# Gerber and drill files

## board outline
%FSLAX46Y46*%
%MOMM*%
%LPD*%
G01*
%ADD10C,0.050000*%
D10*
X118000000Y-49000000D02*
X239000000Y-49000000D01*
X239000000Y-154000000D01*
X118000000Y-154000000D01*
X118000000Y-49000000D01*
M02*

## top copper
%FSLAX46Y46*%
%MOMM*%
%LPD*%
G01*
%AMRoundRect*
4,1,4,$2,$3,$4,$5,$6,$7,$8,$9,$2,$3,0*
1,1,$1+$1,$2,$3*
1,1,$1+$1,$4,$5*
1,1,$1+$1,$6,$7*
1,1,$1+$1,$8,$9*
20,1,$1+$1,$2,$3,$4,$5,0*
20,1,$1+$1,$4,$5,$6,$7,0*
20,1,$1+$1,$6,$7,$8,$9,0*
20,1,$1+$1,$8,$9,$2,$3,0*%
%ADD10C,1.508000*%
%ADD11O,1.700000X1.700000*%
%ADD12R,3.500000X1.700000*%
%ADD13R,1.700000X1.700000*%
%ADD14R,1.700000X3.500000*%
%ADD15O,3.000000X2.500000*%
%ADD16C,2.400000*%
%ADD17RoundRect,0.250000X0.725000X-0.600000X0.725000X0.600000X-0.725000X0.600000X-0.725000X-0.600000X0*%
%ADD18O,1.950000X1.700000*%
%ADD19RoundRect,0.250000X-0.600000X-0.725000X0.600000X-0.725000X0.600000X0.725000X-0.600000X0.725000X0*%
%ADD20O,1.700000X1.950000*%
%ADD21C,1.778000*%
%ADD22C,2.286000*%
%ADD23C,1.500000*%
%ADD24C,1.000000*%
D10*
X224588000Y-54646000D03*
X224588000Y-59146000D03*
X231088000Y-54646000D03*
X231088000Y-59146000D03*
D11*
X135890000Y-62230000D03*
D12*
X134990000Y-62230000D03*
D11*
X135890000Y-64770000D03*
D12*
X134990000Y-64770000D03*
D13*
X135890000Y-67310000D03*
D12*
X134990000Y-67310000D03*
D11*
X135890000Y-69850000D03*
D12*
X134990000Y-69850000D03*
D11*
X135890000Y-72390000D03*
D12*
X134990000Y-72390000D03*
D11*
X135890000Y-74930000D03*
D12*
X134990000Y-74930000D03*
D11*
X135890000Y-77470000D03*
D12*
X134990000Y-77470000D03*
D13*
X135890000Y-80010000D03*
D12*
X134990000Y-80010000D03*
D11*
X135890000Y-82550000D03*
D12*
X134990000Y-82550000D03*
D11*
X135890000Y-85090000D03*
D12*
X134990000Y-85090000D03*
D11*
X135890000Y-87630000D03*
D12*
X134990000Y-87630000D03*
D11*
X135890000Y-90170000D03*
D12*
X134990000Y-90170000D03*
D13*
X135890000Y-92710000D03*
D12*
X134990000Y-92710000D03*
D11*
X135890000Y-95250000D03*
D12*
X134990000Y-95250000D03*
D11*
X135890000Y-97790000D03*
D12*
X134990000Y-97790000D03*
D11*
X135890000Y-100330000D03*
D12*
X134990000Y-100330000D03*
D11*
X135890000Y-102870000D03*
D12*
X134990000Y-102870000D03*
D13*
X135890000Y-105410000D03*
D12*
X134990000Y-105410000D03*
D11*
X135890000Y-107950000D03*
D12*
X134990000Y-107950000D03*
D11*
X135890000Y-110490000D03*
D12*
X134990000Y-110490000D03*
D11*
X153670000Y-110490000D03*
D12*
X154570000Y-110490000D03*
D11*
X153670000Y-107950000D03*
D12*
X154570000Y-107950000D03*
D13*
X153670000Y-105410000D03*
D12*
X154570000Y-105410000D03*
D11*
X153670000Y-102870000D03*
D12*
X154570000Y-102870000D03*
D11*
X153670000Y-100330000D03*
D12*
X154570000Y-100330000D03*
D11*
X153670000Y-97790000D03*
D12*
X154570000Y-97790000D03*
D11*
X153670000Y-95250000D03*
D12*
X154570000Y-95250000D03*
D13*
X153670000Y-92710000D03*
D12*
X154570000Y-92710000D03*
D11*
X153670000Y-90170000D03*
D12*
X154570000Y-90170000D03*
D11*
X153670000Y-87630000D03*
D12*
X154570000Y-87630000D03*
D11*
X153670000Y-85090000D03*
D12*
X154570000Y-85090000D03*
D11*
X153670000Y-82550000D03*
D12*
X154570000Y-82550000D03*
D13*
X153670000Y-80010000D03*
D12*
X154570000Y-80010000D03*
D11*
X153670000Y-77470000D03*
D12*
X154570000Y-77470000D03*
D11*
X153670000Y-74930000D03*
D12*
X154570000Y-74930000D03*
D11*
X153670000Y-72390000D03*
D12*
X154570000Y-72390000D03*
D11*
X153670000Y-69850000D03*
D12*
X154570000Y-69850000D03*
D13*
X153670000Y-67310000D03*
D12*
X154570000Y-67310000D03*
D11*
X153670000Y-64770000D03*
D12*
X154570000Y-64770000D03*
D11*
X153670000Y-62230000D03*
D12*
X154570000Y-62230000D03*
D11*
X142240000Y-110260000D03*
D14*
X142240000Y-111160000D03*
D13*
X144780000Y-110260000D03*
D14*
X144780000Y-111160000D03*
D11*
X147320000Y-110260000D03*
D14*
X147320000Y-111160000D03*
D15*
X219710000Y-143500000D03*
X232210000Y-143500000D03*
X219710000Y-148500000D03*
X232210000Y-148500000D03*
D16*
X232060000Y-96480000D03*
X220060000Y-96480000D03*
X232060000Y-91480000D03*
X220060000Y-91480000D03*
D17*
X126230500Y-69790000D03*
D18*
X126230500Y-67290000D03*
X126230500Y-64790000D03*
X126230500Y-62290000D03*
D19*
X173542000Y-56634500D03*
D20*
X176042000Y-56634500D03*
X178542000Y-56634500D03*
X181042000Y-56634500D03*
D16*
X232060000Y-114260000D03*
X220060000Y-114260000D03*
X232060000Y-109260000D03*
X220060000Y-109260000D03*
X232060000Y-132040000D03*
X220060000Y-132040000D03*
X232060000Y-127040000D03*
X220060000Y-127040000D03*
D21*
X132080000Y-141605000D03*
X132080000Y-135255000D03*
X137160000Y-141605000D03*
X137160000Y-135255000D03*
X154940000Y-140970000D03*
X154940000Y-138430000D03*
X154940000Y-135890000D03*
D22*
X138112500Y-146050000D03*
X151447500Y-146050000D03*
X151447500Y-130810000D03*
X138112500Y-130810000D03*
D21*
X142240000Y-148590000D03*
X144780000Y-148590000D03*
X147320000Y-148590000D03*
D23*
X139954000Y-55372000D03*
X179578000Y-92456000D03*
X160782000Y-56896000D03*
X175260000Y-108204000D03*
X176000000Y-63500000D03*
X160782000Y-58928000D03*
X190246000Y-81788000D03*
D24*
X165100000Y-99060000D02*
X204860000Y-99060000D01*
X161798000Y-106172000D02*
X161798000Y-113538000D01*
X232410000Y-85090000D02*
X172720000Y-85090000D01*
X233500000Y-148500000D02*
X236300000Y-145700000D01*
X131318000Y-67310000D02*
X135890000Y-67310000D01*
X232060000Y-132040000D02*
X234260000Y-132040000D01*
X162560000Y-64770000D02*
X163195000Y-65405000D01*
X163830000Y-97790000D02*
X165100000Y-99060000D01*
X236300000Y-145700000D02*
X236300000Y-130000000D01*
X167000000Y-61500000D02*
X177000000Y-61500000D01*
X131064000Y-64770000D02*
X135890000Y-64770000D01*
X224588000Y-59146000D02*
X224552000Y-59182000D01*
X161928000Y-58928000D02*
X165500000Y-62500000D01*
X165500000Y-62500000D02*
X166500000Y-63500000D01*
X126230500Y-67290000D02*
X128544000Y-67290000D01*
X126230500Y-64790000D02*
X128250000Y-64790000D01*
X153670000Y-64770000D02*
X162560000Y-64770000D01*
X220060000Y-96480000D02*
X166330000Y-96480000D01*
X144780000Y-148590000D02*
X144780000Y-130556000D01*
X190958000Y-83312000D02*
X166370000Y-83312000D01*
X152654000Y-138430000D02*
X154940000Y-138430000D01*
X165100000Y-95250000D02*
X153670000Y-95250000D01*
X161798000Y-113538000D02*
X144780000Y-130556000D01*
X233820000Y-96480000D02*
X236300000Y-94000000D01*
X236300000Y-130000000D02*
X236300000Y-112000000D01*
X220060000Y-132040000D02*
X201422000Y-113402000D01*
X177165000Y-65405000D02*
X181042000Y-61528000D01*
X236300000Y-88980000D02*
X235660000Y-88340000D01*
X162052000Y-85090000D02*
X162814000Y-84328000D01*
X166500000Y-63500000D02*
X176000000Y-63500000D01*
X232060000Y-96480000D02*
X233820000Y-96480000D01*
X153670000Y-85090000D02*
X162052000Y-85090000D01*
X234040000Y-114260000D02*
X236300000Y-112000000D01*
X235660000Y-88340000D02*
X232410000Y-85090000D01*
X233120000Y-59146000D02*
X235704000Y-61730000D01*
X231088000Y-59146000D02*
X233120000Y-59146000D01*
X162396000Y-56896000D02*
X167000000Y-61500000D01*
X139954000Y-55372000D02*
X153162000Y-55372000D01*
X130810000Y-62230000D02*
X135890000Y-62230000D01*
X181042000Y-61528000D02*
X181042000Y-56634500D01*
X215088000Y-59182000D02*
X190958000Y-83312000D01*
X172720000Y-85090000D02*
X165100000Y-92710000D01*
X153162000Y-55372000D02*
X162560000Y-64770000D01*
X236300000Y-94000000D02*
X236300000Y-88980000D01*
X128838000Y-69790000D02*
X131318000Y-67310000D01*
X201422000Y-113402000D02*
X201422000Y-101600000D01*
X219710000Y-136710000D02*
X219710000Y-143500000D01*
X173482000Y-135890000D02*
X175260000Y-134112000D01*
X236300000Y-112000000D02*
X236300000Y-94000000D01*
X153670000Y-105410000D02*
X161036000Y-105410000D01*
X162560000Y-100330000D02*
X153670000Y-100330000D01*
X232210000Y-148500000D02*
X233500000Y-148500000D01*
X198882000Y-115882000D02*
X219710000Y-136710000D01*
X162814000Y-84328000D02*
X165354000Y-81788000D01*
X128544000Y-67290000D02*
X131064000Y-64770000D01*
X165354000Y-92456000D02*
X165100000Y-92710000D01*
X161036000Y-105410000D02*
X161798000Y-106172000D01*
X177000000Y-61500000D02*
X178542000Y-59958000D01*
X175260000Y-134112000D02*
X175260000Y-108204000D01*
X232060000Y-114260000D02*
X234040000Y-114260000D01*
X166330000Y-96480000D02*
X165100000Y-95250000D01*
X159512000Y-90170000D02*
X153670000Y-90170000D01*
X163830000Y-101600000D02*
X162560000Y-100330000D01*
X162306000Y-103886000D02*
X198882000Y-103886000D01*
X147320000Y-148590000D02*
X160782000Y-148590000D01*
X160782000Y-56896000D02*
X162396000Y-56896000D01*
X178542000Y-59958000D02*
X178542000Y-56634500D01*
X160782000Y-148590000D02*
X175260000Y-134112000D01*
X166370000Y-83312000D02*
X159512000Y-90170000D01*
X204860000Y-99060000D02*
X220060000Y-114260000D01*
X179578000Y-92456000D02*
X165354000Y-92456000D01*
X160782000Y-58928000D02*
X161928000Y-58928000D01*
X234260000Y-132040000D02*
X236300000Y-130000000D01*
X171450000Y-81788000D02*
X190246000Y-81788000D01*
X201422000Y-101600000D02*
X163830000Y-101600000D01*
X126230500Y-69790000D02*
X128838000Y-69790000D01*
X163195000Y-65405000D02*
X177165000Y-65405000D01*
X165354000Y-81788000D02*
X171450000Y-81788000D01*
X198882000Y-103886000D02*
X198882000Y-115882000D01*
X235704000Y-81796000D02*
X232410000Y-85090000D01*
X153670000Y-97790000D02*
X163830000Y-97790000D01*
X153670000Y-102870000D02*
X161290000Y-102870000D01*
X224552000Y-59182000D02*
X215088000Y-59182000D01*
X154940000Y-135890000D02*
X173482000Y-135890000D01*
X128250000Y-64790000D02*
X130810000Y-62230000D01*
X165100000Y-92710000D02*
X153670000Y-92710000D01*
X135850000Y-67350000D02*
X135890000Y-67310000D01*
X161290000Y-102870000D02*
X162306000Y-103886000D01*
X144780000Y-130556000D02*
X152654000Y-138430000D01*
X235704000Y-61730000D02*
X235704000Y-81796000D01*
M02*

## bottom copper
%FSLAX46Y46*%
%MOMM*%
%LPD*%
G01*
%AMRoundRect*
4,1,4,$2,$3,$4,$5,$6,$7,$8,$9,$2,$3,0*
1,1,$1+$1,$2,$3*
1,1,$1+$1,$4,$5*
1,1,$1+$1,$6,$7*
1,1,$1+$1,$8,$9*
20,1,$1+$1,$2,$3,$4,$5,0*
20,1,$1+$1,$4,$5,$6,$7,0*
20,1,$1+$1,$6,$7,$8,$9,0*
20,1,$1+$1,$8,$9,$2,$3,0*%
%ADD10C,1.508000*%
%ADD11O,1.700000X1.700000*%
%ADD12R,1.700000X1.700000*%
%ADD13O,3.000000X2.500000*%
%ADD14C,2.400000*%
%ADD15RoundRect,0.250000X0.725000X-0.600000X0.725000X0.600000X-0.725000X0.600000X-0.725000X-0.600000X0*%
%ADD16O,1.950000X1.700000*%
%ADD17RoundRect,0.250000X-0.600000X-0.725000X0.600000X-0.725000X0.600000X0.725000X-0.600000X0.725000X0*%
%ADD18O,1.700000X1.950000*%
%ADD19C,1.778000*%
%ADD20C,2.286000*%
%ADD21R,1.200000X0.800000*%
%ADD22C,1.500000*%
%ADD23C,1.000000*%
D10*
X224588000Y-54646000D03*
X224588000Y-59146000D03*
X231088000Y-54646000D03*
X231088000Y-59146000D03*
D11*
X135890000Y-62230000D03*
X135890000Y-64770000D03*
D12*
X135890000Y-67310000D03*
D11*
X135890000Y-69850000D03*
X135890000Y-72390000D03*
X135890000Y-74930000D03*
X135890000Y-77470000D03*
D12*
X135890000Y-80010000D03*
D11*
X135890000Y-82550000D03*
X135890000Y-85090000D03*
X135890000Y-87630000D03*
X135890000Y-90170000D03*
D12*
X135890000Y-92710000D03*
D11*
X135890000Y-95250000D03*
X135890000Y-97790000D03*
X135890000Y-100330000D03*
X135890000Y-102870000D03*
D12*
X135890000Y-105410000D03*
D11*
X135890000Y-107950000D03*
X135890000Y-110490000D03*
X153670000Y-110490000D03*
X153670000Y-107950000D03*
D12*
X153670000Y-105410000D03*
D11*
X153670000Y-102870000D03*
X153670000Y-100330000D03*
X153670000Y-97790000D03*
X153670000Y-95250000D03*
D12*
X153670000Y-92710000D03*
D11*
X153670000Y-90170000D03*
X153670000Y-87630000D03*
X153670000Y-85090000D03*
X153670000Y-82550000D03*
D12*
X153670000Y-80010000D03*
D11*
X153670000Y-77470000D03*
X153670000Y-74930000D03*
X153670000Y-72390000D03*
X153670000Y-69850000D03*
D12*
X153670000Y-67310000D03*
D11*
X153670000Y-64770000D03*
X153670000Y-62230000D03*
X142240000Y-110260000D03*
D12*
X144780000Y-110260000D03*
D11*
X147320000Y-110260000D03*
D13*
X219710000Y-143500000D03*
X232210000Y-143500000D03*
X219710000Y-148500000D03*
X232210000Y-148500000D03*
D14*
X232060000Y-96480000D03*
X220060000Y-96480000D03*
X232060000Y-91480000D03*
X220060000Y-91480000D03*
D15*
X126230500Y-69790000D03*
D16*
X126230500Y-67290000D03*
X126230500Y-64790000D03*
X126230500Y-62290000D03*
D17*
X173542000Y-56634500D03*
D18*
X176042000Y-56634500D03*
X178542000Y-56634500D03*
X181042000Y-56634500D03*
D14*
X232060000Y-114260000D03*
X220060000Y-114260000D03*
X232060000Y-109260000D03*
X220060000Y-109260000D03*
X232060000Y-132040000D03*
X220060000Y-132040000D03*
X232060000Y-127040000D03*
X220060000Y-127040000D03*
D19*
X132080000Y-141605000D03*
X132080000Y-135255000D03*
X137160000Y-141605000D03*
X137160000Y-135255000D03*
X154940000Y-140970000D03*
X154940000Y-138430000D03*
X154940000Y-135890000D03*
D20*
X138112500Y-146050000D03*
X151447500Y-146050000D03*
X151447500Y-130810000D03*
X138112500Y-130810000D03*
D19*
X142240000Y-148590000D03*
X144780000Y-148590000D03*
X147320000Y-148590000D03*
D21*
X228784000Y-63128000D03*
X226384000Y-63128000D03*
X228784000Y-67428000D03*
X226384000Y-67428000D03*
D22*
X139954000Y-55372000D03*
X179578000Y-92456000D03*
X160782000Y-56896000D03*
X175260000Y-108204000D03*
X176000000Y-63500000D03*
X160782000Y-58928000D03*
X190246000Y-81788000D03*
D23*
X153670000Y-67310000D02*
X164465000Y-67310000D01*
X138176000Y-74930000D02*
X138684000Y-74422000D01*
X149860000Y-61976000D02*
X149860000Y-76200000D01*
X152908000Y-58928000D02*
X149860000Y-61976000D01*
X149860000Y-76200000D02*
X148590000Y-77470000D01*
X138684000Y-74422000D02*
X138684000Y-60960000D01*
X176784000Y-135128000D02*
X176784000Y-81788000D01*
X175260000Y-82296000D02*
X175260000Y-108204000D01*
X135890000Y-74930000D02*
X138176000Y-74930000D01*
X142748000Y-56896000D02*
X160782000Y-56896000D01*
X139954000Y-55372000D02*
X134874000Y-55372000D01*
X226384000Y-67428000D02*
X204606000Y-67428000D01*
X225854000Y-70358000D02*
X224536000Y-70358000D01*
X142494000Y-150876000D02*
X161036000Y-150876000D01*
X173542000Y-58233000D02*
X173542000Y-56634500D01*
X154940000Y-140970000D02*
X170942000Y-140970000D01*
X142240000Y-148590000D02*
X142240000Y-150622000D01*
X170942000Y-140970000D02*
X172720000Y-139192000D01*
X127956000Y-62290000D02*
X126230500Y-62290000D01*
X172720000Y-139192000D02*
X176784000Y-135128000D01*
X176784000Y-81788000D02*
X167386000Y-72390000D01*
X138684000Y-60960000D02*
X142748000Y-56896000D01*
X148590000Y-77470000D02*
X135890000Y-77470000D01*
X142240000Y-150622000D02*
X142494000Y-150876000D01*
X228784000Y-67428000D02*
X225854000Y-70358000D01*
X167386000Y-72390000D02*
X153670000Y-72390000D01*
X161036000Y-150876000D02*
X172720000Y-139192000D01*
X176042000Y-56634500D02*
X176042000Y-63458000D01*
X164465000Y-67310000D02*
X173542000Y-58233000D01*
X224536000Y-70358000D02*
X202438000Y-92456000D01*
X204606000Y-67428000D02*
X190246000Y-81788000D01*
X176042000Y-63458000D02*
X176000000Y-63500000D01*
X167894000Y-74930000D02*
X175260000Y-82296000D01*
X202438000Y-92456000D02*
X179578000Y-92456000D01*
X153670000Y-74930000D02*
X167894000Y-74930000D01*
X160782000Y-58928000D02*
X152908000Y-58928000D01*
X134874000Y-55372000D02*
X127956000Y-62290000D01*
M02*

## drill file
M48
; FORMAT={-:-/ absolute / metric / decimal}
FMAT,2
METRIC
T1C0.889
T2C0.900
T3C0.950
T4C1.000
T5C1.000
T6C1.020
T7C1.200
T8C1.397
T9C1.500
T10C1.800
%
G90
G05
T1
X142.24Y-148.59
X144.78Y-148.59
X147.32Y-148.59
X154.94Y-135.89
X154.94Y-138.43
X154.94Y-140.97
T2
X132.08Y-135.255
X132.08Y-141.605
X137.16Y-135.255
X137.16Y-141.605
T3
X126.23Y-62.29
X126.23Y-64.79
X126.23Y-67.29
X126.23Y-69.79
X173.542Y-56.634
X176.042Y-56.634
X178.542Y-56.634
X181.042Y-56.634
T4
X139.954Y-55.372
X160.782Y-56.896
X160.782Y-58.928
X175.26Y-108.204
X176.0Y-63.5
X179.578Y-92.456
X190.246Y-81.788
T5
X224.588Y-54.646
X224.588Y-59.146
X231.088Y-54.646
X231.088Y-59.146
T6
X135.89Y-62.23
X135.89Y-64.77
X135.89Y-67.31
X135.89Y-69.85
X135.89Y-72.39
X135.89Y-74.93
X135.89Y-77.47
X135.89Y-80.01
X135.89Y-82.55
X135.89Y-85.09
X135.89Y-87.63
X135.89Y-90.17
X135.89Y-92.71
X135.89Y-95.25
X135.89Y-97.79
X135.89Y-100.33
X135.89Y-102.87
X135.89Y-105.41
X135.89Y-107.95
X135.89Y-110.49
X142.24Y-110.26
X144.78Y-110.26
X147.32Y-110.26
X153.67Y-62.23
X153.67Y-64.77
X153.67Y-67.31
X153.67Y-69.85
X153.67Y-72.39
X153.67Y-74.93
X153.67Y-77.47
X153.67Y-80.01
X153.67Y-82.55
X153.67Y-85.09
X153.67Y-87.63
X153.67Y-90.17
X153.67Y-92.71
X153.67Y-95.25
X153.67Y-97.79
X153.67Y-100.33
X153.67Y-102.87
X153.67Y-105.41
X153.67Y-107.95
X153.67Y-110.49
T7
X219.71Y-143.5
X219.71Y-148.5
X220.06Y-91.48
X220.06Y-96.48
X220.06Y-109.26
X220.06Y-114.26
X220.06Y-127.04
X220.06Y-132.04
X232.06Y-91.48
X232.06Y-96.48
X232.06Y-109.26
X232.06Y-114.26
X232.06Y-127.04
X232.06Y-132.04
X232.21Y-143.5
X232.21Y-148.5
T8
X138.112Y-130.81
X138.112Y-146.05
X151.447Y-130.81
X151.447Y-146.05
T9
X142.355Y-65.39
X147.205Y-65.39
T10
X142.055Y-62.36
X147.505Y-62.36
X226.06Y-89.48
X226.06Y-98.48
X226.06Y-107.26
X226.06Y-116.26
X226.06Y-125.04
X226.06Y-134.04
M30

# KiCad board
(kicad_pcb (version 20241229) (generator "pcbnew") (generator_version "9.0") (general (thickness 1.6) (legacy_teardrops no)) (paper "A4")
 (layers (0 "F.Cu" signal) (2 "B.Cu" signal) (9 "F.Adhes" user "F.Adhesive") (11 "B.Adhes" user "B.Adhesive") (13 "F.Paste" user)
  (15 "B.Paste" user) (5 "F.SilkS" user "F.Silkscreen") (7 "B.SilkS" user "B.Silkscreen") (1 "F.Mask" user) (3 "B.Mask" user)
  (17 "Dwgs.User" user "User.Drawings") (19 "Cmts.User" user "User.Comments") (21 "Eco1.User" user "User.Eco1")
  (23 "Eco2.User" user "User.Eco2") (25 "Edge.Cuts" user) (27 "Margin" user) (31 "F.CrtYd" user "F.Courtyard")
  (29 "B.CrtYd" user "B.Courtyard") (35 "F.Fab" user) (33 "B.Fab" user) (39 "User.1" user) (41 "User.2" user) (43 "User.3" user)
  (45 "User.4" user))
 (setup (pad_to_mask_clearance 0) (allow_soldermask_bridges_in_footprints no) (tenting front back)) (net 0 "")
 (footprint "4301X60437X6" (layer "F.Cu") (at 227.838 56.896)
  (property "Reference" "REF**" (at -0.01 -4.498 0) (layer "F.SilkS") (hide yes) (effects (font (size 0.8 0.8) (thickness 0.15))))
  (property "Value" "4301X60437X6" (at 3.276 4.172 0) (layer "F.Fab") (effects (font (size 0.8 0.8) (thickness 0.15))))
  (pad "1" thru_hole circle (at -3.25 -2.25) (size 1.508 1.508) (drill 1) (layers "*.Cu" "*.Mask") (remove_unused_layers no)
   (solder_mask_margin 0.102))
  (pad "2" thru_hole circle (at -3.25 2.25) (size 1.508 1.508) (drill 1) (layers "*.Cu" "*.Mask") (remove_unused_layers no)
   (solder_mask_margin 0.102))
  (pad "3" thru_hole circle (at 3.25 -2.25) (size 1.508 1.508) (drill 1) (layers "*.Cu" "*.Mask") (remove_unused_layers no)
   (solder_mask_margin 0.102))
  (pad "4" thru_hole circle (at 3.25 2.25) (size 1.508 1.508) (drill 1) (layers "*.Cu" "*.Mask") (remove_unused_layers no)
   (solder_mask_margin 0.102)))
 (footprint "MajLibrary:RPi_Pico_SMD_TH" (layer "F.Cu") (at 144.78 86.36)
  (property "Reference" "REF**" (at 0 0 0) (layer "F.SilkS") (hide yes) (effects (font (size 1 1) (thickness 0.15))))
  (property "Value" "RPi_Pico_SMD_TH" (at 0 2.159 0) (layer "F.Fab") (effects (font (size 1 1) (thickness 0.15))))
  (pad "" np_thru_hole oval (at -2.725 -24) (size 1.8 1.8) (drill 1.8) (layers "*.Cu" "*.Mask"))
  (pad "" np_thru_hole oval (at -2.425 -20.97) (size 1.5 1.5) (drill 1.5) (layers "*.Cu" "*.Mask"))
  (pad "" np_thru_hole oval (at 2.425 -20.97) (size 1.5 1.5) (drill 1.5) (layers "*.Cu" "*.Mask"))
  (pad "" np_thru_hole oval (at 2.725 -24) (size 1.8 1.8) (drill 1.8) (layers "*.Cu" "*.Mask"))
  (pad "1" thru_hole oval (at -8.89 -24.13) (size 1.7 1.7) (drill 1.02) (layers "*.Cu" "*.Mask") (remove_unused_layers no))
  (pad "1" smd rect (at -8.89 -24.13) (size 3.5 1.7) (drill (offset -0.9 0)) (layers "F.Cu" "F.Mask"))
  (pad "2" thru_hole oval (at -8.89 -21.59) (size 1.7 1.7) (drill 1.02) (layers "*.Cu" "*.Mask") (remove_unused_layers no))
  (pad "2" smd rect (at -8.89 -21.59) (size 3.5 1.7) (drill (offset -0.9 0)) (layers "F.Cu" "F.Mask"))
  (pad "3" thru_hole rect (at -8.89 -19.05) (size 1.7 1.7) (drill 1.02) (layers "*.Cu" "*.Mask") (remove_unused_layers no))
  (pad "3" smd rect (at -8.89 -19.05) (size 3.5 1.7) (drill (offset -0.9 0)) (layers "F.Cu" "F.Mask"))
  (pad "4" thru_hole oval (at -8.89 -16.51) (size 1.7 1.7) (drill 1.02) (layers "*.Cu" "*.Mask") (remove_unused_layers no))
  (pad "4" smd rect (at -8.89 -16.51) (size 3.5 1.7) (drill (offset -0.9 0)) (layers "F.Cu" "F.Mask"))
  (pad "5" thru_hole oval (at -8.89 -13.97) (size 1.7 1.7) (drill 1.02) (layers "*.Cu" "*.Mask") (remove_unused_layers no))
  (pad "5" smd rect (at -8.89 -13.97) (size 3.5 1.7) (drill (offset -0.9 0)) (layers "F.Cu" "F.Mask"))
  (pad "6" thru_hole oval (at -8.89 -11.43) (size 1.7 1.7) (drill 1.02) (layers "*.Cu" "*.Mask") (remove_unused_layers no))
  (pad "6" smd rect (at -8.89 -11.43) (size 3.5 1.7) (drill (offset -0.9 0)) (layers "F.Cu" "F.Mask"))
  (pad "7" thru_hole oval (at -8.89 -8.89) (size 1.7 1.7) (drill 1.02) (layers "*.Cu" "*.Mask") (remove_unused_layers no))
  (pad "7" smd rect (at -8.89 -8.89) (size 3.5 1.7) (drill (offset -0.9 0)) (layers "F.Cu" "F.Mask"))
  (pad "8" thru_hole rect (at -8.89 -6.35) (size 1.7 1.7) (drill 1.02) (layers "*.Cu" "*.Mask") (remove_unused_layers no))
  (pad "8" smd rect (at -8.89 -6.35) (size 3.5 1.7) (drill (offset -0.9 0)) (layers "F.Cu" "F.Mask"))
  (pad "9" thru_hole oval (at -8.89 -3.81) (size 1.7 1.7) (drill 1.02) (layers "*.Cu" "*.Mask") (remove_unused_layers no))
  (pad "9" smd rect (at -8.89 -3.81) (size 3.5 1.7) (drill (offset -0.9 0)) (layers "F.Cu" "F.Mask"))
  (pad "10" thru_hole oval (at -8.89 -1.27) (size 1.7 1.7) (drill 1.02) (layers "*.Cu" "*.Mask") (remove_unused_layers no))
  (pad "10" smd rect (at -8.89 -1.27) (size 3.5 1.7) (drill (offset -0.9 0)) (layers "F.Cu" "F.Mask"))
  (pad "11" thru_hole oval (at -8.89 1.27) (size 1.7 1.7) (drill 1.02) (layers "*.Cu" "*.Mask") (remove_unused_layers no))
  (pad "11" smd rect (at -8.89 1.27) (size 3.5 1.7) (drill (offset -0.9 0)) (layers "F.Cu" "F.Mask"))
  (pad "12" thru_hole oval (at -8.89 3.81) (size 1.7 1.7) (drill 1.02) (layers "*.Cu" "*.Mask") (remove_unused_layers no))
  (pad "12" smd rect (at -8.89 3.81) (size 3.5 1.7) (drill (offset -0.9 0)) (layers "F.Cu" "F.Mask"))
  (pad "13" thru_hole rect (at -8.89 6.35) (size 1.7 1.7) (drill 1.02) (layers "*.Cu" "*.Mask") (remove_unused_layers no))
  (pad "13" smd rect (at -8.89 6.35) (size 3.5 1.7) (drill (offset -0.9 0)) (layers "F.Cu" "F.Mask"))
  (pad "14" thru_hole oval (at -8.89 8.89) (size 1.7 1.7) (drill 1.02) (layers "*.Cu" "*.Mask") (remove_unused_layers no))
  (pad "14" smd rect (at -8.89 8.89) (size 3.5 1.7) (drill (offset -0.9 0)) (layers "F.Cu" "F.Mask"))
  (pad "15" thru_hole oval (at -8.89 11.43) (size 1.7 1.7) (drill 1.02) (layers "*.Cu" "*.Mask") (remove_unused_layers no))
  (pad "15" smd rect (at -8.89 11.43) (size 3.5 1.7) (drill (offset -0.9 0)) (layers "F.Cu" "F.Mask"))
  (pad "16" thru_hole oval (at -8.89 13.97) (size 1.7 1.7) (drill 1.02) (layers "*.Cu" "*.Mask") (remove_unused_layers no))
  (pad "16" smd rect (at -8.89 13.97) (size 3.5 1.7) (drill (offset -0.9 0)) (layers "F.Cu" "F.Mask"))
  (pad "17" thru_hole oval (at -8.89 16.51) (size 1.7 1.7) (drill 1.02) (layers "*.Cu" "*.Mask") (remove_unused_layers no))
  (pad "17" smd rect (at -8.89 16.51) (size 3.5 1.7) (drill (offset -0.9 0)) (layers "F.Cu" "F.Mask"))
  (pad "18" thru_hole rect (at -8.89 19.05) (size 1.7 1.7) (drill 1.02) (layers "*.Cu" "*.Mask") (remove_unused_layers no))
  (pad "18" smd rect (at -8.89 19.05) (size 3.5 1.7) (drill (offset -0.9 0)) (layers "F.Cu" "F.Mask"))
  (pad "19" thru_hole oval (at -8.89 21.59) (size 1.7 1.7) (drill 1.02) (layers "*.Cu" "*.Mask") (remove_unused_layers no))
  (pad "19" smd rect (at -8.89 21.59) (size 3.5 1.7) (drill (offset -0.9 0)) (layers "F.Cu" "F.Mask"))
  (pad "20" thru_hole oval (at -8.89 24.13) (size 1.7 1.7) (drill 1.02) (layers "*.Cu" "*.Mask") (remove_unused_layers no))
  (pad "20" smd rect (at -8.89 24.13) (size 3.5 1.7) (drill (offset -0.9 0)) (layers "F.Cu" "F.Mask"))
  (pad "21" thru_hole oval (at 8.89 24.13) (size 1.7 1.7) (drill 1.02) (layers "*.Cu" "*.Mask") (remove_unused_layers no))
  (pad "21" smd rect (at 8.89 24.13) (size 3.5 1.7) (drill (offset 0.9 0)) (layers "F.Cu" "F.Mask"))
  (pad "22" thru_hole oval (at 8.89 21.59) (size 1.7 1.7) (drill 1.02) (layers "*.Cu" "*.Mask") (remove_unused_layers no))
  (pad "22" smd rect (at 8.89 21.59) (size 3.5 1.7) (drill (offset 0.9 0)) (layers "F.Cu" "F.Mask"))
  (pad "23" thru_hole rect (at 8.89 19.05) (size 1.7 1.7) (drill 1.02) (layers "*.Cu" "*.Mask") (remove_unused_layers no))
  (pad "23" smd rect (at 8.89 19.05) (size 3.5 1.7) (drill (offset 0.9 0)) (layers "F.Cu" "F.Mask"))
  (pad "24" thru_hole oval (at 8.89 16.51) (size 1.7 1.7) (drill 1.02) (layers "*.Cu" "*.Mask") (remove_unused_layers no))
  (pad "24" smd rect (at 8.89 16.51) (size 3.5 1.7) (drill (offset 0.9 0)) (layers "F.Cu" "F.Mask"))
  (pad "25" thru_hole oval (at 8.89 13.97) (size 1.7 1.7) (drill 1.02) (layers "*.Cu" "*.Mask") (remove_unused_layers no))
  (pad "25" smd rect (at 8.89 13.97) (size 3.5 1.7) (drill (offset 0.9 0)) (layers "F.Cu" "F.Mask"))
  (pad "26" thru_hole oval (at 8.89 11.43) (size 1.7 1.7) (drill 1.02) (layers "*.Cu" "*.Mask") (remove_unused_layers no))
  (pad "26" smd rect (at 8.89 11.43) (size 3.5 1.7) (drill (offset 0.9 0)) (layers "F.Cu" "F.Mask"))
  (pad "27" thru_hole oval (at 8.89 8.89) (size 1.7 1.7) (drill 1.02) (layers "*.Cu" "*.Mask") (remove_unused_layers no))
  (pad "27" smd rect (at 8.89 8.89) (size 3.5 1.7) (drill (offset 0.9 0)) (layers "F.Cu" "F.Mask"))
  (pad "28" thru_hole rect (at 8.89 6.35) (size 1.7 1.7) (drill 1.02) (layers "*.Cu" "*.Mask") (remove_unused_layers no))
  (pad "28" smd rect (at 8.89 6.35) (size 3.5 1.7) (drill (offset 0.9 0)) (layers "F.Cu" "F.Mask"))
  (pad "29" thru_hole oval (at 8.89 3.81) (size 1.7 1.7) (drill 1.02) (layers "*.Cu" "*.Mask") (remove_unused_layers no))
  (pad "29" smd rect (at 8.89 3.81) (size 3.5 1.7) (drill (offset 0.9 0)) (layers "F.Cu" "F.Mask"))
  (pad "30" thru_hole oval (at 8.89 1.27) (size 1.7 1.7) (drill 1.02) (layers "*.Cu" "*.Mask") (remove_unused_layers no))
  (pad "30" smd rect (at 8.89 1.27) (size 3.5 1.7) (drill (offset 0.9 0)) (layers "F.Cu" "F.Mask"))
  (pad "31" thru_hole oval (at 8.89 -1.27) (size 1.7 1.7) (drill 1.02) (layers "*.Cu" "*.Mask") (remove_unused_layers no))
  (pad "31" smd rect (at 8.89 -1.27) (size 3.5 1.7) (drill (offset 0.9 0)) (layers "F.Cu" "F.Mask"))
  (pad "32" thru_hole oval (at 8.89 -3.81) (size 1.7 1.7) (drill 1.02) (layers "*.Cu" "*.Mask") (remove_unused_layers no))
  (pad "32" smd rect (at 8.89 -3.81) (size 3.5 1.7) (drill (offset 0.9 0)) (layers "F.Cu" "F.Mask"))
  (pad "33" thru_hole rect (at 8.89 -6.35) (size 1.7 1.7) (drill 1.02) (layers "*.Cu" "*.Mask") (remove_unused_layers no))
  (pad "33" smd rect (at 8.89 -6.35) (size 3.5 1.7) (drill (offset 0.9 0)) (layers "F.Cu" "F.Mask"))
  (pad "34" thru_hole oval (at 8.89 -8.89) (size 1.7 1.7) (drill 1.02) (layers "*.Cu" "*.Mask") (remove_unused_layers no))
  (pad "34" smd rect (at 8.89 -8.89) (size 3.5 1.7) (drill (offset 0.9 0)) (layers "F.Cu" "F.Mask"))
  (pad "35" thru_hole oval (at 8.89 -11.43) (size 1.7 1.7) (drill 1.02) (layers "*.Cu" "*.Mask") (remove_unused_layers no))
  (pad "35" smd rect (at 8.89 -11.43) (size 3.5 1.7) (drill (offset 0.9 0)) (layers "F.Cu" "F.Mask"))
  (pad "36" thru_hole oval (at 8.89 -13.97) (size 1.7 1.7) (drill 1.02) (layers "*.Cu" "*.Mask") (remove_unused_layers no))
  (pad "36" smd rect (at 8.89 -13.97) (size 3.5 1.7) (drill (offset 0.9 0)) (layers "F.Cu" "F.Mask"))
  (pad "37" thru_hole oval (at 8.89 -16.51) (size 1.7 1.7) (drill 1.02) (layers "*.Cu" "*.Mask") (remove_unused_layers no))
  (pad "37" smd rect (at 8.89 -16.51) (size 3.5 1.7) (drill (offset 0.9 0)) (layers "F.Cu" "F.Mask"))
  (pad "38" thru_hole rect (at 8.89 -19.05) (size 1.7 1.7) (drill 1.02) (layers "*.Cu" "*.Mask") (remove_unused_layers no))
  (pad "38" smd rect (at 8.89 -19.05) (size 3.5 1.7) (drill (offset 0.9 0)) (layers "F.Cu" "F.Mask"))
  (pad "39" thru_hole oval (at 8.89 -21.59) (size 1.7 1.7) (drill 1.02) (layers "*.Cu" "*.Mask") (remove_unused_layers no))
  (pad "39" smd rect (at 8.89 -21.59) (size 3.5 1.7) (drill (offset 0.9 0)) (layers "F.Cu" "F.Mask"))
  (pad "40" thru_hole oval (at 8.89 -24.13) (size 1.7 1.7) (drill 1.02) (layers "*.Cu" "*.Mask") (remove_unused_layers no))
  (pad "40" smd rect (at 8.89 -24.13) (size 3.5 1.7) (drill (offset 0.9 0)) (layers "F.Cu" "F.Mask"))
  (pad "41" thru_hole oval (at -2.54 23.9) (size 1.7 1.7) (drill 1.02) (layers "*.Cu" "*.Mask") (remove_unused_layers no))
  (pad "41" smd rect (at -2.54 23.9 90) (size 3.5 1.7) (drill (offset -0.9 0)) (layers "F.Cu" "F.Mask"))
  (pad "42" thru_hole rect (at 0 23.9) (size 1.7 1.7) (drill 1.02) (layers "*.Cu" "*.Mask") (remove_unused_layers no))
  (pad "42" smd rect (at 0 23.9 90) (size 3.5 1.7) (drill (offset -0.9 0)) (layers "F.Cu" "F.Mask"))
  (pad "43" thru_hole oval (at 2.54 23.9) (size 1.7 1.7) (drill 1.02) (layers "*.Cu" "*.Mask") (remove_unused_layers no))
  (pad "43" smd rect (at 2.54 23.9 90) (size 3.5 1.7) (drill (offset -0.9 0)) (layers "F.Cu" "F.Mask")))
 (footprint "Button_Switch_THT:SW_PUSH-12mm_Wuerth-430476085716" (layer "F.Cu") (at 219.71 143.5)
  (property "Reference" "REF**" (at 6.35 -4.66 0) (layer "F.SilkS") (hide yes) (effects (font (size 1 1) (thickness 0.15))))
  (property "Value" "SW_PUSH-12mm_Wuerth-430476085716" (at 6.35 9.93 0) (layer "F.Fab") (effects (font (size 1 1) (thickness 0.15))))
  (pad "1" thru_hole oval (at 0 0) (size 3 2.5) (drill 1.2) (layers "*.Cu" "*.Mask") (remove_unused_layers no))
  (pad "1" thru_hole oval (at 12.5 0) (size 3 2.5) (drill 1.2) (layers "*.Cu" "*.Mask") (remove_unused_layers no))
  (pad "2" thru_hole oval (at 0 5) (size 3 2.5) (drill 1.2) (layers "*.Cu" "*.Mask") (remove_unused_layers no))
  (pad "2" thru_hole oval (at 12.5 5) (size 3 2.5) (drill 1.2) (layers "*.Cu" "*.Mask") (remove_unused_layers no)))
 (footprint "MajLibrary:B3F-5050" (layer "F.Cu") (at 226.06 93.98)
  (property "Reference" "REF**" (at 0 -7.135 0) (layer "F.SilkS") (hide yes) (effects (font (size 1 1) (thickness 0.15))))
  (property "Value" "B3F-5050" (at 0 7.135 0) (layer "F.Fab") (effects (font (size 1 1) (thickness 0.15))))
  (pad "" np_thru_hole circle (at 0 -4.5) (size 1.8 1.8) (drill 1.8) (layers "*.Cu" "*.Mask"))
  (pad "" np_thru_hole circle (at 0 4.5) (size 1.8 1.8) (drill 1.8) (layers "*.Cu" "*.Mask"))
  (pad "1" thru_hole circle (at 6 2.5) (size 2.4 2.4) (drill 1.2) (layers "*.Cu" "*.Mask") (remove_unused_layers no)
   (solder_mask_margin 0.102))
  (pad "2" thru_hole circle (at -6 2.5) (size 2.4 2.4) (drill 1.2) (layers "*.Cu" "*.Mask") (remove_unused_layers no)
   (solder_mask_margin 0.102))
  (pad "3" thru_hole circle (at 6 -2.5) (size 2.4 2.4) (drill 1.2) (layers "*.Cu" "*.Mask") (remove_unused_layers no)
   (solder_mask_margin 0.102))
  (pad "4" thru_hole circle (at -6 -2.5) (size 2.4 2.4) (drill 1.2) (layers "*.Cu" "*.Mask") (remove_unused_layers no)
   (solder_mask_margin 0.102)))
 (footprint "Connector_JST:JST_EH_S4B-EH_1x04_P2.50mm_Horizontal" (layer "F.Cu") (at 126.2305 69.79 90)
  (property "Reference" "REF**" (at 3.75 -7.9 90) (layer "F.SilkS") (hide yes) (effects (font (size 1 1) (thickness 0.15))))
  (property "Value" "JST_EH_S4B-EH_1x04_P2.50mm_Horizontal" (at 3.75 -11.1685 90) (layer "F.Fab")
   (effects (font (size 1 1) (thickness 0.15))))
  (pad "1" thru_hole roundrect (at 0 0 90) (size 1.7 1.95) (drill 0.95) (layers "*.Cu" "*.Mask") (remove_unused_layers no)
   (roundrect_rratio 0.147059))
  (pad "2" thru_hole oval (at 2.5 0 90) (size 1.7 1.95) (drill 0.95) (layers "*.Cu" "*.Mask") (remove_unused_layers no))
  (pad "3" thru_hole oval (at 5 0 90) (size 1.7 1.95) (drill 0.95) (layers "*.Cu" "*.Mask") (remove_unused_layers no))
  (pad "4" thru_hole oval (at 7.5 0 90) (size 1.7 1.95) (drill 0.95) (layers "*.Cu" "*.Mask") (remove_unused_layers no)))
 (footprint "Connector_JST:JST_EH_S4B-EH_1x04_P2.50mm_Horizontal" (layer "F.Cu") (at 173.542 56.6345)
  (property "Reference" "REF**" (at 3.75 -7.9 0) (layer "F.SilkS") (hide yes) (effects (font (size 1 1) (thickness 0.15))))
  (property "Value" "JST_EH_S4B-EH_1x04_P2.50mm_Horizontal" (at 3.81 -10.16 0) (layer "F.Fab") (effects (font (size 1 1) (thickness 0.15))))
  (pad "1" thru_hole roundrect (at 0 0) (size 1.7 1.95) (drill 0.95) (layers "*.Cu" "*.Mask") (remove_unused_layers no)
   (roundrect_rratio 0.147059))
  (pad "2" thru_hole oval (at 2.5 0) (size 1.7 1.95) (drill 0.95) (layers "*.Cu" "*.Mask") (remove_unused_layers no))
  (pad "3" thru_hole oval (at 5 0) (size 1.7 1.95) (drill 0.95) (layers "*.Cu" "*.Mask") (remove_unused_layers no))
  (pad "4" thru_hole oval (at 7.5 0) (size 1.7 1.95) (drill 0.95) (layers "*.Cu" "*.Mask") (remove_unused_layers no)))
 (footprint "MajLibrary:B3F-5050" (layer "F.Cu") (at 226.06 111.76)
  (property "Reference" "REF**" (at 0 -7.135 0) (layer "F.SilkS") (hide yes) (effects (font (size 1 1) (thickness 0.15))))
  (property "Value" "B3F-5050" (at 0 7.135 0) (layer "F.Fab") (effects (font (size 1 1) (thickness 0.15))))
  (pad "" np_thru_hole circle (at 0 -4.5) (size 1.8 1.8) (drill 1.8) (layers "*.Cu" "*.Mask"))
  (pad "" np_thru_hole circle (at 0 4.5) (size 1.8 1.8) (drill 1.8) (layers "*.Cu" "*.Mask"))
  (pad "1" thru_hole circle (at 6 2.5) (size 2.4 2.4) (drill 1.2) (layers "*.Cu" "*.Mask") (remove_unused_layers no)
   (solder_mask_margin 0.102))
  (pad "2" thru_hole circle (at -6 2.5) (size 2.4 2.4) (drill 1.2) (layers "*.Cu" "*.Mask") (remove_unused_layers no)
   (solder_mask_margin 0.102))
  (pad "3" thru_hole circle (at 6 -2.5) (size 2.4 2.4) (drill 1.2) (layers "*.Cu" "*.Mask") (remove_unused_layers no)
   (solder_mask_margin 0.102))
  (pad "4" thru_hole circle (at -6 -2.5) (size 2.4 2.4) (drill 1.2) (layers "*.Cu" "*.Mask") (remove_unused_layers no)
   (solder_mask_margin 0.102)))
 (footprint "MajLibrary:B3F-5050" (layer "F.Cu") (at 226.06 129.54)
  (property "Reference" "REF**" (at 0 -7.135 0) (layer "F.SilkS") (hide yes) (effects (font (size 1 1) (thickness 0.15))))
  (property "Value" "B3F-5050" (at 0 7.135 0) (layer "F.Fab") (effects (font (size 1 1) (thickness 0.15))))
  (pad "" np_thru_hole circle (at 0 -4.5) (size 1.8 1.8) (drill 1.8) (layers "*.Cu" "*.Mask"))
  (pad "" np_thru_hole circle (at 0 4.5) (size 1.8 1.8) (drill 1.8) (layers "*.Cu" "*.Mask"))
  (pad "1" thru_hole circle (at 6 2.5) (size 2.4 2.4) (drill 1.2) (layers "*.Cu" "*.Mask") (remove_unused_layers no)
   (solder_mask_margin 0.102))
  (pad "2" thru_hole circle (at -6 2.5) (size 2.4 2.4) (drill 1.2) (layers "*.Cu" "*.Mask") (remove_unused_layers no)
   (solder_mask_margin 0.102))
  (pad "3" thru_hole circle (at 6 -2.5) (size 2.4 2.4) (drill 1.2) (layers "*.Cu" "*.Mask") (remove_unused_layers no)
   (solder_mask_margin 0.102))
  (pad "4" thru_hole circle (at -6 -2.5) (size 2.4 2.4) (drill 1.2) (layers "*.Cu" "*.Mask") (remove_unused_layers no)
   (solder_mask_margin 0.102)))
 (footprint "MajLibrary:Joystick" (layer "F.Cu") (at 144.78 138.43 90)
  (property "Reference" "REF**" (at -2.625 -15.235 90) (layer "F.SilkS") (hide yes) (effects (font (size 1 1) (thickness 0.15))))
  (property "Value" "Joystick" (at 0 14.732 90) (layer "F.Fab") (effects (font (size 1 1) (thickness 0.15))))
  (pad "B1A" thru_hole circle (at -3.175 -12.7 90) (size 1.778 1.778) (drill 0.9) (layers "*.Cu" "*.Mask") (remove_unused_layers no)
   (solder_mask_margin 0.102))
  (pad "B1B" thru_hole circle (at 3.175 -12.7 90) (size 1.778 1.778) (drill 0.9) (layers "*.Cu" "*.Mask") (remove_unused_layers no)
   (solder_mask_margin 0.102))
  (pad "B2A" thru_hole circle (at -3.175 -7.62 90) (size 1.778 1.778) (drill 0.9) (layers "*.Cu" "*.Mask") (remove_unused_layers no)
   (solder_mask_margin 0.102))
  (pad "B2B" thru_hole circle (at 3.175 -7.62 90) (size 1.778 1.778) (drill 0.9) (layers "*.Cu" "*.Mask") (remove_unused_layers no)
   (solder_mask_margin 0.102))
  (pad "H1" thru_hole circle (at -2.54 10.16 90) (size 1.778 1.778) (drill 0.889) (layers "*.Cu" "*.Mask") (remove_unused_layers no)
   (solder_mask_margin 0.102))
  (pad "H2" thru_hole circle (at 0 10.16 90) (size 1.778 1.778) (drill 0.889) (layers "*.Cu" "*.Mask") (remove_unused_layers no)
   (solder_mask_margin 0.102))
  (pad "H3" thru_hole circle (at 2.54 10.16 90) (size 1.778 1.778) (drill 0.889) (layers "*.Cu" "*.Mask") (remove_unused_layers no)
   (solder_mask_margin 0.102))
  (pad "S1" thru_hole circle (at -7.62 -6.6675 90) (size 2.286 2.286) (drill 1.397) (layers "*.Cu" "*.Mask") (remove_unused_layers no)
   (solder_mask_margin 0.102))
  (pad "S2" thru_hole circle (at -7.62 6.6675 90) (size 2.286 2.286) (drill 1.397) (layers "*.Cu" "*.Mask") (remove_unused_layers no)
   (solder_mask_margin 0.102))
  (pad "S3" thru_hole circle (at 7.62 6.6675 90) (size 2.286 2.286) (drill 1.397) (layers "*.Cu" "*.Mask") (remove_unused_layers no)
   (solder_mask_margin 0.102))
  (pad "S4" thru_hole circle (at 7.62 -6.6675 90) (size 2.286 2.286) (drill 1.397) (layers "*.Cu" "*.Mask") (remove_unused_layers no)
   (solder_mask_margin 0.102))
  (pad "V1" thru_hole circle (at -10.16 -2.54 90) (size 1.778 1.778) (drill 0.889) (layers "*.Cu" "*.Mask") (remove_unused_layers no)
   (solder_mask_margin 0.102))
  (pad "V2" thru_hole circle (at -10.16 0 90) (size 1.778 1.778) (drill 0.889) (layers "*.Cu" "*.Mask") (remove_unused_layers no)
   (solder_mask_margin 0.102))
  (pad "V3" thru_hole circle (at -10.16 2.54 90) (size 1.778 1.778) (drill 0.889) (layers "*.Cu" "*.Mask") (remove_unused_layers no)
   (solder_mask_margin 0.102)))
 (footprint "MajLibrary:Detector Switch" (layer "B.Cu") (at 227.584 65.278 180)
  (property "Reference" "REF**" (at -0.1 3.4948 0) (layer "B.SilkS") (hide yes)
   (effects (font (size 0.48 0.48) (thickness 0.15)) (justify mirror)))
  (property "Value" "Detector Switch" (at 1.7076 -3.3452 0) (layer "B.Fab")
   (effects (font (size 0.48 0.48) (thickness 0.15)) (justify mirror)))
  (pad "1" smd rect (at -1.2 2.15 180) (size 1.2 0.8) (layers "B.Cu" "B.Mask" "B.Paste") (solder_mask_margin 0.102))
  (pad "2" smd rect (at 1.2 2.15 180) (size 1.2 0.8) (layers "B.Cu" "B.Mask" "B.Paste") (solder_mask_margin 0.102))
  (pad "3" smd rect (at -1.2 -2.15 180) (size 1.2 0.8) (layers "B.Cu" "B.Mask" "B.Paste") (solder_mask_margin 0.102))
  (pad "4" smd rect (at 1.2 -2.15 180) (size 1.2 0.8) (layers "B.Cu" "B.Mask" "B.Paste") (solder_mask_margin 0.102)))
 (gr_rect (start 118 49) (end 239 154) (stroke (width 0.05) (type default)) (fill no) (layer "Edge.Cuts"))
 (segment (start 165.1 99.06) (end 204.86 99.06) (width 1) (layer "F.Cu") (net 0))
 (segment (start 161.798 106.172) (end 161.798 113.538) (width 1) (layer "F.Cu") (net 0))
 (segment (start 232.41 85.09) (end 172.72 85.09) (width 1) (layer "F.Cu") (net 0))
 (segment (start 233.5 148.5) (end 236.3 145.7) (width 1) (layer "F.Cu") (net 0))
 (segment (start 131.318 67.31) (end 135.89 67.31) (width 1) (layer "F.Cu") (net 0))
 (segment (start 232.06 132.04) (end 234.26 132.04) (width 1) (layer "F.Cu") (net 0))
 (segment (start 162.56 64.77) (end 163.195 65.405) (width 1) (layer "F.Cu") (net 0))
 (segment (start 163.83 97.79) (end 165.1 99.06) (width 1) (layer "F.Cu") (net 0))
 (segment (start 236.3 145.7) (end 236.3 130) (width 1) (layer "F.Cu") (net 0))
 (segment (start 167 61.5) (end 177 61.5) (width 1) (layer "F.Cu") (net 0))
 (segment (start 131.064 64.77) (end 135.89 64.77) (width 1) (layer "F.Cu") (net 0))
 (segment (start 224.588 59.146) (end 224.552 59.182) (width 1) (layer "F.Cu") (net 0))
 (segment (start 161.928 58.928) (end 165.5 62.5) (width 1) (layer "F.Cu") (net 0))
 (segment (start 165.5 62.5) (end 166.5 63.5) (width 1) (layer "F.Cu") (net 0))
 (segment (start 126.2305 67.29) (end 128.544 67.29) (width 1) (layer "F.Cu") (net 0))
 (segment (start 126.2305 64.79) (end 128.25 64.79) (width 1) (layer "F.Cu") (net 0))
 (segment (start 153.67 64.77) (end 162.56 64.77) (width 1) (layer "F.Cu") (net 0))
 (segment (start 220.06 96.48) (end 166.33 96.48) (width 1) (layer "F.Cu") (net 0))
 (segment (start 144.78 148.59) (end 144.78 130.556) (width 1) (layer "F.Cu") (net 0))
 (segment (start 190.958 83.312) (end 166.37 83.312) (width 1) (layer "F.Cu") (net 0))
 (segment (start 152.654 138.43) (end 154.94 138.43) (width 1) (layer "F.Cu") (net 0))
 (segment (start 165.1 95.25) (end 153.67 95.25) (width 1) (layer "F.Cu") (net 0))
 (segment (start 161.798 113.538) (end 144.78 130.556) (width 1) (layer "F.Cu") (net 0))
 (segment (start 233.82 96.48) (end 236.3 94) (width 1) (layer "F.Cu") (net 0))
 (segment (start 236.3 130) (end 236.3 112) (width 1) (layer "F.Cu") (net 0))
 (segment (start 220.06 132.04) (end 201.422 113.402) (width 1) (layer "F.Cu") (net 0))
 (segment (start 177.165 65.405) (end 181.042 61.528) (width 1) (layer "F.Cu") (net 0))
 (segment (start 236.3 88.98) (end 235.66 88.34) (width 1) (layer "F.Cu") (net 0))
 (segment (start 162.052 85.09) (end 162.814 84.328) (width 1) (layer "F.Cu") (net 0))
 (segment (start 166.5 63.5) (end 176 63.5) (width 1) (layer "F.Cu") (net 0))
 (segment (start 232.06 96.48) (end 233.82 96.48) (width 1) (layer "F.Cu") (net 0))
 (segment (start 153.67 85.09) (end 162.052 85.09) (width 1) (layer "F.Cu") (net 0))
 (segment (start 234.04 114.26) (end 236.3 112) (width 1) (layer "F.Cu") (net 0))
 (segment (start 235.66 88.34) (end 232.41 85.09) (width 1) (layer "F.Cu") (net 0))
 (segment (start 233.12 59.146) (end 235.704 61.73) (width 1) (layer "F.Cu") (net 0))
 (segment (start 231.088 59.146) (end 233.12 59.146) (width 1) (layer "F.Cu") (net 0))
 (segment (start 162.396 56.896) (end 167 61.5) (width 1) (layer "F.Cu") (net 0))
 (segment (start 139.954 55.372) (end 153.162 55.372) (width 1) (layer "F.Cu") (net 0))
 (segment (start 130.81 62.23) (end 135.89 62.23) (width 1) (layer "F.Cu") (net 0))
 (segment (start 181.042 61.528) (end 181.042 56.6345) (width 1) (layer "F.Cu") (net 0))
 (segment (start 215.088 59.182) (end 190.958 83.312) (width 1) (layer "F.Cu") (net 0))
 (segment (start 172.72 85.09) (end 165.1 92.71) (width 1) (layer "F.Cu") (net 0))
 (segment (start 153.162 55.372) (end 162.56 64.77) (width 1) (layer "F.Cu") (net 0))
 (segment (start 236.3 94) (end 236.3 88.98) (width 1) (layer "F.Cu") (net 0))
 (segment (start 128.838 69.79) (end 131.318 67.31) (width 1) (layer "F.Cu") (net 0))
 (segment (start 201.422 113.402) (end 201.422 101.6) (width 1) (layer "F.Cu") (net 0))
 (segment (start 219.71 136.71) (end 219.71 143.5) (width 1) (layer "F.Cu") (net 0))
 (segment (start 173.482 135.89) (end 175.26 134.112) (width 1) (layer "F.Cu") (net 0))
 (segment (start 236.3 112) (end 236.3 94) (width 1) (layer "F.Cu") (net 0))
 (segment (start 153.67 105.41) (end 161.036 105.41) (width 1) (layer "F.Cu") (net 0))
 (segment (start 162.56 100.33) (end 153.67 100.33) (width 1) (layer "F.Cu") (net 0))
 (segment (start 232.21 148.5) (end 233.5 148.5) (width 1) (layer "F.Cu") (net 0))
 (segment (start 198.882 115.882) (end 219.71 136.71) (width 1) (layer "F.Cu") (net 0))
 (segment (start 162.814 84.328) (end 165.354 81.788) (width 1) (layer "F.Cu") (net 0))
 (segment (start 128.544 67.29) (end 131.064 64.77) (width 1) (layer "F.Cu") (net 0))
 (segment (start 165.354 92.456) (end 165.1 92.71) (width 1) (layer "F.Cu") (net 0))
 (segment (start 161.036 105.41) (end 161.798 106.172) (width 1) (layer "F.Cu") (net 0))
 (segment (start 177 61.5) (end 178.542 59.958) (width 1) (layer "F.Cu") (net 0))
 (segment (start 175.26 134.112) (end 175.26 108.204) (width 1) (layer "F.Cu") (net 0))
 (segment (start 232.06 114.26) (end 234.04 114.26) (width 1) (layer "F.Cu") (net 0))
 (segment (start 166.33 96.48) (end 165.1 95.25) (width 1) (layer "F.Cu") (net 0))
 (segment (start 159.512 90.17) (end 153.67 90.17) (width 1) (layer "F.Cu") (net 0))
 (segment (start 163.83 101.6) (end 162.56 100.33) (width 1) (layer "F.Cu") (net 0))
 (segment (start 162.306 103.886) (end 198.882 103.886) (width 1) (layer "F.Cu") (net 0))
 (segment (start 147.32 148.59) (end 160.782 148.59) (width 1) (layer "F.Cu") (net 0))
 (segment (start 160.782 56.896) (end 162.396 56.896) (width 1) (layer "F.Cu") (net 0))
 (segment (start 178.542 59.958) (end 178.542 56.6345) (width 1) (layer "F.Cu") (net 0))
 (segment (start 160.782 148.59) (end 175.26 134.112) (width 1) (layer "F.Cu") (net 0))
 (segment (start 166.37 83.312) (end 159.512 90.17) (width 1) (layer "F.Cu") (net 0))
 (segment (start 204.86 99.06) (end 220.06 114.26) (width 1) (layer "F.Cu") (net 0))
 (segment (start 179.578 92.456) (end 165.354 92.456) (width 1) (layer "F.Cu") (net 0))
 (segment (start 160.782 58.928) (end 161.928 58.928) (width 1) (layer "F.Cu") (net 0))
 (segment (start 234.26 132.04) (end 236.3 130) (width 1) (layer "F.Cu") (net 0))
 (segment (start 171.45 81.788) (end 190.246 81.788) (width 1) (layer "F.Cu") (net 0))
 (segment (start 201.422 101.6) (end 163.83 101.6) (width 1) (layer "F.Cu") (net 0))
 (segment (start 126.2305 69.79) (end 128.838 69.79) (width 1) (layer "F.Cu") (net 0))
 (segment (start 163.195 65.405) (end 177.165 65.405) (width 1) (layer "F.Cu") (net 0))
 (segment (start 165.354 81.788) (end 171.45 81.788) (width 1) (layer "F.Cu") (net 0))
 (segment (start 198.882 103.886) (end 198.882 115.882) (width 1) (layer "F.Cu") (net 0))
 (segment (start 235.704 81.796) (end 232.41 85.09) (width 1) (layer "F.Cu") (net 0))
 (segment (start 153.67 97.79) (end 163.83 97.79) (width 1) (layer "F.Cu") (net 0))
 (segment (start 153.67 102.87) (end 161.29 102.87) (width 1) (layer "F.Cu") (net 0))
 (segment (start 224.552 59.182) (end 215.088 59.182) (width 1) (layer "F.Cu") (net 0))
 (segment (start 154.94 135.89) (end 173.482 135.89) (width 1) (layer "F.Cu") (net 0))
 (segment (start 128.25 64.79) (end 130.81 62.23) (width 1) (layer "F.Cu") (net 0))
 (segment (start 165.1 92.71) (end 153.67 92.71) (width 1) (layer "F.Cu") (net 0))
 (segment (start 135.85 67.35) (end 135.89 67.31) (width 1) (layer "F.Cu") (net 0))
 (segment (start 161.29 102.87) (end 162.306 103.886) (width 1) (layer "F.Cu") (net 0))
 (segment (start 144.78 130.556) (end 152.654 138.43) (width 1) (layer "F.Cu") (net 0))
 (segment (start 235.704 61.73) (end 235.704 81.796) (width 1) (layer "F.Cu") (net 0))
 (via (at 139.954 55.372) (size 1.5) (drill 1) (layers "F.Cu" "B.Cu") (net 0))
 (via (at 179.578 92.456) (size 1.5) (drill 1) (layers "F.Cu" "B.Cu") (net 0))
 (via (at 160.782 56.896) (size 1.5) (drill 1) (layers "F.Cu" "B.Cu") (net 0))
 (via (at 175.26 108.204) (size 1.5) (drill 1) (layers "F.Cu" "B.Cu") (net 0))
 (via (at 176 63.5) (size 1.5) (drill 1) (layers "F.Cu" "B.Cu") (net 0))
 (via (at 160.782 58.928) (size 1.5) (drill 1) (layers "F.Cu" "B.Cu") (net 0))
 (via (at 190.246 81.788) (size 1.5) (drill 1) (layers "F.Cu" "B.Cu") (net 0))
 (segment (start 153.67 67.31) (end 164.465 67.31) (width 1) (layer "B.Cu") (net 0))
 (segment (start 138.176 74.93) (end 138.684 74.422) (width 1) (layer "B.Cu") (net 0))
 (segment (start 149.86 61.976) (end 149.86 76.2) (width 1) (layer "B.Cu") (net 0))
 (segment (start 152.908 58.928) (end 149.86 61.976) (width 1) (layer "B.Cu") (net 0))
 (segment (start 149.86 76.2) (end 148.59 77.47) (width 1) (layer "B.Cu") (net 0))
 (segment (start 138.684 74.422) (end 138.684 60.96) (width 1) (layer "B.Cu") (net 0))
 (segment (start 176.784 135.128) (end 176.784 81.788) (width 1) (layer "B.Cu") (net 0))
 (segment (start 175.26 82.296) (end 175.26 108.204) (width 1) (layer "B.Cu") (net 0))
 (segment (start 135.89 74.93) (end 138.176 74.93) (width 1) (layer "B.Cu") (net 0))
 (segment (start 142.748 56.896) (end 160.782 56.896) (width 1) (layer "B.Cu") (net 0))
 (segment (start 139.954 55.372) (end 134.874 55.372) (width 1) (layer "B.Cu") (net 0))
 (segment (start 226.384 67.428) (end 204.606 67.428) (width 1) (layer "B.Cu") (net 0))
 (segment (start 225.854 70.358) (end 224.536 70.358) (width 1) (layer "B.Cu") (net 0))
 (segment (start 142.494 150.876) (end 161.036 150.876) (width 1) (layer "B.Cu") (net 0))
 (segment (start 173.542 58.233) (end 173.542 56.6345) (width 1) (layer "B.Cu") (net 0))
 (segment (start 154.94 140.97) (end 170.942 140.97) (width 1) (layer "B.Cu") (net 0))
 (segment (start 142.24 148.59) (end 142.24 150.622) (width 1) (layer "B.Cu") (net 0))
 (segment (start 170.942 140.97) (end 172.72 139.192) (width 1) (layer "B.Cu") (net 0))
 (segment (start 127.956 62.29) (end 126.2305 62.29) (width 1) (layer "B.Cu") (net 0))
 (segment (start 172.72 139.192) (end 176.784 135.128) (width 1) (layer "B.Cu") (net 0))
 (segment (start 176.784 81.788) (end 167.386 72.39) (width 1) (layer "B.Cu") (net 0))
 (segment (start 138.684 60.96) (end 142.748 56.896) (width 1) (layer "B.Cu") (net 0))
 (segment (start 148.59 77.47) (end 135.89 77.47) (width 1) (layer "B.Cu") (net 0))
 (segment (start 142.24 150.622) (end 142.494 150.876) (width 1) (layer "B.Cu") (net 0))
 (segment (start 228.784 67.428) (end 225.854 70.358) (width 1) (layer "B.Cu") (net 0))
 (segment (start 167.386 72.39) (end 153.67 72.39) (width 1) (layer "B.Cu") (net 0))
 (segment (start 161.036 150.876) (end 172.72 139.192) (width 1) (layer "B.Cu") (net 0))
 (segment (start 176.042 56.6345) (end 176.042 63.458) (width 1) (layer "B.Cu") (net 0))
 (segment (start 164.465 67.31) (end 173.542 58.233) (width 1) (layer "B.Cu") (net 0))
 (segment (start 224.536 70.358) (end 202.438 92.456) (width 1) (layer "B.Cu") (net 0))
 (segment (start 204.606 67.428) (end 190.246 81.788) (width 1) (layer "B.Cu") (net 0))
 (segment (start 176.042 63.458) (end 176 63.5) (width 1) (layer "B.Cu") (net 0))
 (segment (start 167.894 74.93) (end 175.26 82.296) (width 1) (layer "B.Cu") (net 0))
 (segment (start 202.438 92.456) (end 179.578 92.456) (width 1) (layer "B.Cu") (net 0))
 (segment (start 153.67 74.93) (end 167.894 74.93) (width 1) (layer "B.Cu") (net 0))
 (segment (start 160.782 58.928) (end 152.908 58.928) (width 1) (layer "B.Cu") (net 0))
 (segment (start 134.874 55.372) (end 127.956 62.29) (width 1) (layer "B.Cu") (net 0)))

